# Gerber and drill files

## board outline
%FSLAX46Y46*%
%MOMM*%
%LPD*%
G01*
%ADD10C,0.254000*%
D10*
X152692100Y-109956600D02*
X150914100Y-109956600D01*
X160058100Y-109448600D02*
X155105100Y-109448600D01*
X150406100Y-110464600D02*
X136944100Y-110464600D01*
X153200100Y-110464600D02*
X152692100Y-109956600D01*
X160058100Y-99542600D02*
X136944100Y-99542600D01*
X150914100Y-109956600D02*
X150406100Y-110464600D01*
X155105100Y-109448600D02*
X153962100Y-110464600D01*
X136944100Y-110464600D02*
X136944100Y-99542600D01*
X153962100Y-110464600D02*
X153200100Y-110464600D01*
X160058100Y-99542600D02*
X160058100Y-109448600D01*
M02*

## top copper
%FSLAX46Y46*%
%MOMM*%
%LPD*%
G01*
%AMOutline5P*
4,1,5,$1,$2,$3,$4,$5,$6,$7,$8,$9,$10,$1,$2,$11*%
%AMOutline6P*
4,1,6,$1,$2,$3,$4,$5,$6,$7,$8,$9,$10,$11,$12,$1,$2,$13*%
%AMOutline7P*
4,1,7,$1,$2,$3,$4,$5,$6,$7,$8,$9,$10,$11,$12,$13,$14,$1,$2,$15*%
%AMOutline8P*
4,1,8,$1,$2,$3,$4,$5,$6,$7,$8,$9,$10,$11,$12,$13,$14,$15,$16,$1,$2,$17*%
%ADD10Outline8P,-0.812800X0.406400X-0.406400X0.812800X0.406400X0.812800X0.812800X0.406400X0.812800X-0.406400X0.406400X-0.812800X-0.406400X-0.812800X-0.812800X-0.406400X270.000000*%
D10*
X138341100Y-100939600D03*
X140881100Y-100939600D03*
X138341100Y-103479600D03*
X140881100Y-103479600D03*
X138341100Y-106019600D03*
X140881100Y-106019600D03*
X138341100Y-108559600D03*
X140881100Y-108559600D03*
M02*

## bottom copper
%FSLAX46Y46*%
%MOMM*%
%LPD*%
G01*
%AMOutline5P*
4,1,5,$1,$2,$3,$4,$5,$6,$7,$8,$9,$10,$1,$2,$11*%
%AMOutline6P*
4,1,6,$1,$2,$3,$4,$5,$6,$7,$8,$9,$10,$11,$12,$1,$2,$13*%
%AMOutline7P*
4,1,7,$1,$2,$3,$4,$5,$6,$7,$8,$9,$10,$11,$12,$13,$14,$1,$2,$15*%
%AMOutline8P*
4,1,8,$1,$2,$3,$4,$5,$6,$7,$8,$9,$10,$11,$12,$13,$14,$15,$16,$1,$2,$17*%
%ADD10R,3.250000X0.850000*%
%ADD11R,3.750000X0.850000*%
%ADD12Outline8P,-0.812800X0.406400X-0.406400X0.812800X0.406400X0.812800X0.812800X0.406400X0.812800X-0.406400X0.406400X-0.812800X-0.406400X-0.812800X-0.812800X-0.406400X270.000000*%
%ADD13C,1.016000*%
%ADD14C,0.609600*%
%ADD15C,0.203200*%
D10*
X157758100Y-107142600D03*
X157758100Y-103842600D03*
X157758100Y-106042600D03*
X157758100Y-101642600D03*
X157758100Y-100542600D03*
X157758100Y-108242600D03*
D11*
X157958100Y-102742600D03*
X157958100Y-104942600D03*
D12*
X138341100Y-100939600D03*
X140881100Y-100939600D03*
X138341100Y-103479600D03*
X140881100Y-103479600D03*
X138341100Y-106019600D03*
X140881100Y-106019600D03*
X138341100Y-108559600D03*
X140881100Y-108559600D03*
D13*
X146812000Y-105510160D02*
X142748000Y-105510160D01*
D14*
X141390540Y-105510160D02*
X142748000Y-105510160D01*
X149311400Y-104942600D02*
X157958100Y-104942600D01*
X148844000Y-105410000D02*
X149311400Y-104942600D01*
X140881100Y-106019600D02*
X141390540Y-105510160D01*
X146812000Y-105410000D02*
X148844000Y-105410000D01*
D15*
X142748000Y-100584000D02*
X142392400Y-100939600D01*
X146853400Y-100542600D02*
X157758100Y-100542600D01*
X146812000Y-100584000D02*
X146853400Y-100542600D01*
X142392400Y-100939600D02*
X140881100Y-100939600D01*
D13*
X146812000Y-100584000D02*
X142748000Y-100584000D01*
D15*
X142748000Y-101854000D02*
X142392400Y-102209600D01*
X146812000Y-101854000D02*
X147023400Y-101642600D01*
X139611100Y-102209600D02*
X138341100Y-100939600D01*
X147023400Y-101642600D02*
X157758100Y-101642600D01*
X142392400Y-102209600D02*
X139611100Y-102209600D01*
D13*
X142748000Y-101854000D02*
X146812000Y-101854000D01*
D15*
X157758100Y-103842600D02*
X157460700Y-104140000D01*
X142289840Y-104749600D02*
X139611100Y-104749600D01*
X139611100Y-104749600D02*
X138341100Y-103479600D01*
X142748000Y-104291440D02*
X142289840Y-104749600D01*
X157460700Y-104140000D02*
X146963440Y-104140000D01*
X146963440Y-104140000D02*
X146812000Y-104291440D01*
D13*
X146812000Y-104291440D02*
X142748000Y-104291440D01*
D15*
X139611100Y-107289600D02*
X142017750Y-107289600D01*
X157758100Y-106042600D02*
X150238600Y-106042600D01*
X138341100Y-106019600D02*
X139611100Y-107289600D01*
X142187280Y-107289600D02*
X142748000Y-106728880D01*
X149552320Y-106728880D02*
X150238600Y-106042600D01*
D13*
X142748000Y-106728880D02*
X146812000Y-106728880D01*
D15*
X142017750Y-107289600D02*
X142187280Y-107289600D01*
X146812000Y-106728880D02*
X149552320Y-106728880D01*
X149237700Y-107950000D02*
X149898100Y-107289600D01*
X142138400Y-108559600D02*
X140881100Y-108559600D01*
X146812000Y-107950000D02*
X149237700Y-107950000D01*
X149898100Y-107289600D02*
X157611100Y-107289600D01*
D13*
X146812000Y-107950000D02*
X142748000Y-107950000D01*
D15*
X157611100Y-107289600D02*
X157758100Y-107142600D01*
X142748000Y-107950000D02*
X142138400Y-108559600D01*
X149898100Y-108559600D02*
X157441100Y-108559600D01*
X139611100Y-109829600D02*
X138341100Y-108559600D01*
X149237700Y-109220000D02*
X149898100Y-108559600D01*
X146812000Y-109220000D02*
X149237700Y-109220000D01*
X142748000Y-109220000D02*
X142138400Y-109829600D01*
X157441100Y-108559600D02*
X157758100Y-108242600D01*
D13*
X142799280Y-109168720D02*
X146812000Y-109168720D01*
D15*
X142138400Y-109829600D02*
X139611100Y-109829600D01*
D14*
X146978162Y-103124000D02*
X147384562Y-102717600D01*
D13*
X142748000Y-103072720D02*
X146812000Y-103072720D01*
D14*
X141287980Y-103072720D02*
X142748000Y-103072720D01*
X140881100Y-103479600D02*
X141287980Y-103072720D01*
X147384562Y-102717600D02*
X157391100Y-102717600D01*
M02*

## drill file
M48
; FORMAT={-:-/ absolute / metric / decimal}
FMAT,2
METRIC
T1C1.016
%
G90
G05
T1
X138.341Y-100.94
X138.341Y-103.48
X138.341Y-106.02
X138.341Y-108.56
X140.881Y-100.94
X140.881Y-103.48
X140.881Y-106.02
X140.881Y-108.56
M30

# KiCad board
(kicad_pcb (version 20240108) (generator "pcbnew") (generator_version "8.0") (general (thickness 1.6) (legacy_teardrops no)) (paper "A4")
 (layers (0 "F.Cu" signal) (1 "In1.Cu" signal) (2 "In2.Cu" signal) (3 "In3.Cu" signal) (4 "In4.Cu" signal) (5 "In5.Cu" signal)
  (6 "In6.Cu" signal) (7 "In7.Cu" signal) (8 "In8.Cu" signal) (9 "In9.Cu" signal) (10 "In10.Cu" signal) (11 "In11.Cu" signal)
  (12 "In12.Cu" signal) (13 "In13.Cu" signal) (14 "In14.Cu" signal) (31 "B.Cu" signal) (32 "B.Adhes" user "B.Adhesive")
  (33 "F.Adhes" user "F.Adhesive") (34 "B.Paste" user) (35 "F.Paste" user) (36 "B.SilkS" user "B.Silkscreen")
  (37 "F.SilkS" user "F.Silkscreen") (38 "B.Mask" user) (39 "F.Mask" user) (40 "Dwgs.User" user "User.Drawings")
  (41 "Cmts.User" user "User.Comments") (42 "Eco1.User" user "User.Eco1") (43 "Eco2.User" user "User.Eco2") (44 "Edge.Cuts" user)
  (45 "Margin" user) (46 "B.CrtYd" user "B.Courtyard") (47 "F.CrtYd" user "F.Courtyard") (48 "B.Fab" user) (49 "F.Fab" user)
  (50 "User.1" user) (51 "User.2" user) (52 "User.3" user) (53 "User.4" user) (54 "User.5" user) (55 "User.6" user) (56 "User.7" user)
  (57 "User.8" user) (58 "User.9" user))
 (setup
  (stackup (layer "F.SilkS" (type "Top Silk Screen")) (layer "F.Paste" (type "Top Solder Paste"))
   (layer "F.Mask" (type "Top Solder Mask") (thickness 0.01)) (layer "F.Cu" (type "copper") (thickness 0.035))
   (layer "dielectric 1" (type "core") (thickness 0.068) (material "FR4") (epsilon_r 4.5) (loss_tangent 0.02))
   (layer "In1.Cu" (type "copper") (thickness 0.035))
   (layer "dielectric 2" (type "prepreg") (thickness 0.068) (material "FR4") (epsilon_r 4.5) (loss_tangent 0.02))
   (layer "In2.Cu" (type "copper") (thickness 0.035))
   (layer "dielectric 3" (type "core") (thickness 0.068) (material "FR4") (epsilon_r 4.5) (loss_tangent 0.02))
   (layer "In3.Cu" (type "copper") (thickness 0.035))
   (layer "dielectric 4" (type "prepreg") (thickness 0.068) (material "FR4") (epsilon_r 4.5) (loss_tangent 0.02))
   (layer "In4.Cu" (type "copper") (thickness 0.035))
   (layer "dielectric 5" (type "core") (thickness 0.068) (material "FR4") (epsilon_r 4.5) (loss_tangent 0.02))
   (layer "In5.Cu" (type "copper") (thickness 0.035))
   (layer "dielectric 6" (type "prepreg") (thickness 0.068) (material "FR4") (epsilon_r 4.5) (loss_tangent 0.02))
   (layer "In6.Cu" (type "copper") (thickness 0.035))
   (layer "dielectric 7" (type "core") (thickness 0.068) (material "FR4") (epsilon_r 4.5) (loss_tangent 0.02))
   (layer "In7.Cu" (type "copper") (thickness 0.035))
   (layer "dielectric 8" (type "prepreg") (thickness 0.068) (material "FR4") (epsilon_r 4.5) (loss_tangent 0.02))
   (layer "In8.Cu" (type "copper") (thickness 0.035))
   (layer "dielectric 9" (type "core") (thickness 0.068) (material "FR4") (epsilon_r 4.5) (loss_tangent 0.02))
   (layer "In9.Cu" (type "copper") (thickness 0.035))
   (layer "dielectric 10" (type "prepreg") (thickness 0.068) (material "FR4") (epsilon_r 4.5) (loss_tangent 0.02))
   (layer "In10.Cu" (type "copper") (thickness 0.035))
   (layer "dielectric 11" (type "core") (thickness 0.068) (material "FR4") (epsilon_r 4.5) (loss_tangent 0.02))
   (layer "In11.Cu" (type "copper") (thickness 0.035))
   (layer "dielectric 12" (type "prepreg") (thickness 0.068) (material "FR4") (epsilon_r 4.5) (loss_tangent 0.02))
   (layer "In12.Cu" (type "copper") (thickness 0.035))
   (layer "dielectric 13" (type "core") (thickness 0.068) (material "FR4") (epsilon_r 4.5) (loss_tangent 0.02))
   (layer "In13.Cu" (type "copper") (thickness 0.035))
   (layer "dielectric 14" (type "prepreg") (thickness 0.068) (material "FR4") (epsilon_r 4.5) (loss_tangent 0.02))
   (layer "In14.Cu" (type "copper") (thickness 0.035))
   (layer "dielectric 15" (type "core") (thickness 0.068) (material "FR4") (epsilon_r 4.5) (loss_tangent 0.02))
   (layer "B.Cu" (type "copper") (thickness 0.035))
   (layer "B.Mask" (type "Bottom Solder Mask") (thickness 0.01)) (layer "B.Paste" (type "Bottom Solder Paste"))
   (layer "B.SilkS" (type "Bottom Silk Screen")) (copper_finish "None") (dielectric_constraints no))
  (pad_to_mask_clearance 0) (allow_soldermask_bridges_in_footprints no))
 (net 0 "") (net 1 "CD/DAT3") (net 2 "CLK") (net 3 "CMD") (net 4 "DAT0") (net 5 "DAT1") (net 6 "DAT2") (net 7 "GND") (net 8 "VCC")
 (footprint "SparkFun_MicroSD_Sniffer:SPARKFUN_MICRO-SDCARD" (layer "F.Cu") (at 160.0581 109.7026 90)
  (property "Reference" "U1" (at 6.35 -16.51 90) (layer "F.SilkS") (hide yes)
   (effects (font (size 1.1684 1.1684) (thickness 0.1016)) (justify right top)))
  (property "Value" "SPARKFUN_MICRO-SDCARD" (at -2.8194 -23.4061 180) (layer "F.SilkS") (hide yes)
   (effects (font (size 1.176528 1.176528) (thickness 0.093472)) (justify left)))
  (pad "CD/DAT3" smd rect (at 2.56 -2.3 90) (size 0.85 3.25) (layers "B.Cu" "B.Paste" "B.Mask") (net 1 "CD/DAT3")
   (solder_mask_margin 0.1016))
  (pad "CLK" smd rect (at 5.86 -2.3 90) (size 0.85 3.25) (layers "B.Cu" "B.Paste" "B.Mask") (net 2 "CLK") (solder_mask_margin 0.1016))
  (pad "CMD" smd rect (at 3.66 -2.3 90) (size 0.85 3.25) (layers "B.Cu" "B.Paste" "B.Mask") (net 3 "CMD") (solder_mask_margin 0.1016))
  (pad "DAT0" smd rect (at 8.06 -2.3 90) (size 0.85 3.25) (layers "B.Cu" "B.Paste" "B.Mask") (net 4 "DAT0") (solder_mask_margin 0.1016))
  (pad "DAT1" smd rect (at 9.16 -2.3 90) (size 0.85 3.25) (layers "B.Cu" "B.Paste" "B.Mask") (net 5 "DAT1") (solder_mask_margin 0.1016))
  (pad "DAT2" smd rect (at 1.46 -2.3 90) (size 0.85 3.25) (layers "B.Cu" "B.Paste" "B.Mask") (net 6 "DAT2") (solder_mask_margin 0.1016))
  (pad "GND" smd rect (at 6.96 -2.1 270) (size 0.85 3.75) (layers "B.Cu" "B.Paste" "B.Mask") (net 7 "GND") (solder_mask_margin 0.1016))
  (pad "VCC" smd rect (at 4.76 -2.1 90) (size 0.85 3.75) (layers "B.Cu" "B.Paste" "B.Mask") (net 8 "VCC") (solder_mask_margin 0.1016)))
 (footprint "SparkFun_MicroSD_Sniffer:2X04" (layer "F.Cu") (at 139.6111 104.7496 -90)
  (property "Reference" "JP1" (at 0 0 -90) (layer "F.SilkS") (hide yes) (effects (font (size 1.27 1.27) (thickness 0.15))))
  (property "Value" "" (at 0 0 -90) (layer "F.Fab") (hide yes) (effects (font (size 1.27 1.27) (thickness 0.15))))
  (pad "1" thru_hole roundrect (at -3.81 1.27 270) (size 1.6256 1.6256) (drill 1.016) (layers "*.Cu" "*.Mask") (remove_unused_layers no)
   (roundrect_rratio 0.25) (chamfer_ratio 0.25) (chamfer top_left top_right bottom_left bottom_right) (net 4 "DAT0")
   (solder_mask_margin 0.1016))
  (pad "2" thru_hole roundrect (at -3.81 -1.27 270) (size 1.6256 1.6256) (drill 1.016) (layers "*.Cu" "*.Mask") (remove_unused_layers no)
   (roundrect_rratio 0.25) (chamfer_ratio 0.25) (chamfer top_left top_right bottom_left bottom_right) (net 5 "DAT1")
   (solder_mask_margin 0.1016))
  (pad "3" thru_hole roundrect (at -1.27 1.27 270) (size 1.6256 1.6256) (drill 1.016) (layers "*.Cu" "*.Mask") (remove_unused_layers no)
   (roundrect_rratio 0.25) (chamfer_ratio 0.25) (chamfer top_left top_right bottom_left bottom_right) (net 2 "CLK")
   (solder_mask_margin 0.1016))
  (pad "4" thru_hole roundrect (at -1.27 -1.27 270) (size 1.6256 1.6256) (drill 1.016) (layers "*.Cu" "*.Mask") (remove_unused_layers no)
   (roundrect_rratio 0.25) (chamfer_ratio 0.25) (chamfer top_left top_right bottom_left bottom_right) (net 7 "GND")
   (solder_mask_margin 0.1016))
  (pad "5" thru_hole roundrect (at 1.27 1.27 270) (size 1.6256 1.6256) (drill 1.016) (layers "*.Cu" "*.Mask") (remove_unused_layers no)
   (roundrect_rratio 0.25) (chamfer_ratio 0.25) (chamfer top_left top_right bottom_left bottom_right) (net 3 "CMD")
   (solder_mask_margin 0.1016))
  (pad "6" thru_hole roundrect (at 1.27 -1.27 270) (size 1.6256 1.6256) (drill 1.016) (layers "*.Cu" "*.Mask") (remove_unused_layers no)
   (roundrect_rratio 0.25) (chamfer_ratio 0.25) (chamfer top_left top_right bottom_left bottom_right) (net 8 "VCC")
   (solder_mask_margin 0.1016))
  (pad "7" thru_hole roundrect (at 3.81 1.27 270) (size 1.6256 1.6256) (drill 1.016) (layers "*.Cu" "*.Mask") (remove_unused_layers no)
   (roundrect_rratio 0.25) (chamfer_ratio 0.25) (chamfer top_left top_right bottom_left bottom_right) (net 6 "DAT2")
   (solder_mask_margin 0.1016))
  (pad "8" thru_hole roundrect (at 3.81 -1.27 270) (size 1.6256 1.6256) (drill 1.016) (layers "*.Cu" "*.Mask") (remove_unused_layers no)
   (roundrect_rratio 0.25) (chamfer_ratio 0.25) (chamfer top_left top_right bottom_left bottom_right) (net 1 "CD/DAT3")
   (solder_mask_margin 0.1016)))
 (gr_line (start 152.6921 109.9566) (end 150.9141 109.9566) (stroke (width 0.254) (type solid)) (layer "Edge.Cuts"))
 (gr_line (start 160.0581 109.4486) (end 155.1051 109.4486) (stroke (width 0.254) (type solid)) (layer "Edge.Cuts"))
 (gr_line (start 150.4061 110.4646) (end 136.9441 110.4646) (stroke (width 0.254) (type solid)) (layer "Edge.Cuts"))
 (gr_line (start 153.2001 110.4646) (end 152.6921 109.9566) (stroke (width 0.254) (type solid)) (layer "Edge.Cuts"))
 (gr_line (start 160.0581 99.5426) (end 136.9441 99.5426) (stroke (width 0.254) (type solid)) (layer "Edge.Cuts"))
 (gr_line (start 150.9141 109.9566) (end 150.4061 110.4646) (stroke (width 0.254) (type solid)) (layer "Edge.Cuts"))
 (gr_line (start 155.1051 109.4486) (end 153.9621 110.4646) (stroke (width 0.254) (type solid)) (layer "Edge.Cuts"))
 (gr_line (start 136.9441 110.4646) (end 136.9441 99.5426) (stroke (width 0.254) (type solid)) (layer "Edge.Cuts"))
 (gr_line (start 153.9621 110.4646) (end 153.2001 110.4646) (stroke (width 0.254) (type solid)) (layer "Edge.Cuts"))
 (gr_line (start 160.0581 99.5426) (end 160.0581 109.4486) (stroke (width 0.254) (type solid)) (layer "Edge.Cuts"))
 (segment (start 146.812 105.51016) (end 142.748 105.51016) (width 1.016) (layer "B.Cu") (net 8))
 (segment (start 141.39054 105.51016) (end 142.748 105.51016) (width 0.6096) (layer "B.Cu") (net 8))
 (segment (start 149.3114 104.9426) (end 157.9581 104.9426) (width 0.6096) (layer "B.Cu") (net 8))
 (segment (start 148.844 105.41) (end 149.3114 104.9426) (width 0.6096) (layer "B.Cu") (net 8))
 (segment (start 140.8811 106.0196) (end 141.39054 105.51016) (width 0.6096) (layer "B.Cu") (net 8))
 (segment (start 146.812 105.41) (end 148.844 105.41) (width 0.6096) (layer "B.Cu") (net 8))
 (segment (start 142.748 100.584) (end 142.3924 100.9396) (width 0.2032) (layer "B.Cu") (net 5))
 (segment (start 146.8534 100.5426) (end 157.7581 100.5426) (width 0.2032) (layer "B.Cu") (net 5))
 (segment (start 146.812 100.584) (end 146.8534 100.5426) (width 0.2032) (layer "B.Cu") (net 5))
 (segment (start 142.3924 100.9396) (end 140.8811 100.9396) (width 0.2032) (layer "B.Cu") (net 5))
 (segment (start 146.812 100.584) (end 142.748 100.584) (width 1.016) (layer "B.Cu") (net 5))
 (segment (start 142.748 101.854) (end 142.3924 102.2096) (width 0.2032) (layer "B.Cu") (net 4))
 (segment (start 146.812 101.854) (end 147.0234 101.6426) (width 0.2032) (layer "B.Cu") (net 4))
 (segment (start 139.6111 102.2096) (end 138.3411 100.9396) (width 0.2032) (layer "B.Cu") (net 4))
 (segment (start 147.0234 101.6426) (end 157.7581 101.6426) (width 0.2032) (layer "B.Cu") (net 4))
 (segment (start 142.3924 102.2096) (end 139.6111 102.2096) (width 0.2032) (layer "B.Cu") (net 4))
 (segment (start 142.748 101.854) (end 146.812 101.854) (width 1.016) (layer "B.Cu") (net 4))
 (segment (start 157.7581 103.8426) (end 157.4607 104.14) (width 0.2032) (layer "B.Cu") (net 2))
 (segment (start 142.28984 104.7496) (end 139.6111 104.7496) (width 0.2032) (layer "B.Cu") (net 2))
 (segment (start 139.6111 104.7496) (end 138.3411 103.4796) (width 0.2032) (layer "B.Cu") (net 2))
 (segment (start 142.748 104.29144) (end 142.28984 104.7496) (width 0.2032) (layer "B.Cu") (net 2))
 (segment (start 157.4607 104.14) (end 146.96344 104.14) (width 0.2032) (layer "B.Cu") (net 2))
 (segment (start 146.96344 104.14) (end 146.812 104.29144) (width 0.2032) (layer "B.Cu") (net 2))
 (segment (start 146.812 104.29144) (end 142.748 104.29144) (width 1.016) (layer "B.Cu") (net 2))
 (segment (start 139.6111 107.2896) (end 142.01775 107.2896) (width 0.2032) (layer "B.Cu") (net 3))
 (segment (start 157.7581 106.0426) (end 150.2386 106.0426) (width 0.2032) (layer "B.Cu") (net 3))
 (segment (start 138.3411 106.0196) (end 139.6111 107.2896) (width 0.2032) (layer "B.Cu") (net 3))
 (segment (start 142.18728 107.2896) (end 142.748 106.72888) (width 0.2032) (layer "B.Cu") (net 3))
 (segment (start 149.55232 106.72888) (end 150.2386 106.0426) (width 0.2032) (layer "B.Cu") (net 3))
 (segment (start 142.748 106.72888) (end 146.812 106.72888) (width 1.016) (layer "B.Cu") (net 3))
 (segment (start 142.01775 107.2896) (end 142.18728 107.2896) (width 0.2032) (layer "B.Cu") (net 3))
 (segment (start 146.812 106.72888) (end 149.55232 106.72888) (width 0.2032) (layer "B.Cu") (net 3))
 (segment (start 149.2377 107.95) (end 149.8981 107.2896) (width 0.2032) (layer "B.Cu") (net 1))
 (segment (start 142.1384 108.5596) (end 140.8811 108.5596) (width 0.2032) (layer "B.Cu") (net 1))
 (segment (start 146.812 107.95) (end 149.2377 107.95) (width 0.2032) (layer "B.Cu") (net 1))
 (segment (start 149.8981 107.2896) (end 157.6111 107.2896) (width 0.2032) (layer "B.Cu") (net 1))
 (segment (start 146.812 107.95) (end 142.748 107.95) (width 1.016) (layer "B.Cu") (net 1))
 (segment (start 157.6111 107.2896) (end 157.7581 107.1426) (width 0.2032) (layer "B.Cu") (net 1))
 (segment (start 142.748 107.95) (end 142.1384 108.5596) (width 0.2032) (layer "B.Cu") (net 1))
 (segment (start 149.8981 108.5596) (end 157.4411 108.5596) (width 0.2032) (layer "B.Cu") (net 6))
 (segment (start 139.6111 109.8296) (end 138.3411 108.5596) (width 0.2032) (layer "B.Cu") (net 6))
 (segment (start 149.2377 109.22) (end 149.8981 108.5596) (width 0.2032) (layer "B.Cu") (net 6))
 (segment (start 146.812 109.22) (end 149.2377 109.22) (width 0.2032) (layer "B.Cu") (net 6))
 (segment (start 142.748 109.22) (end 142.1384 109.8296) (width 0.2032) (layer "B.Cu") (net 6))
 (segment (start 157.4411 108.5596) (end 157.7581 108.2426) (width 0.2032) (layer "B.Cu") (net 6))
 (segment (start 142.79928 109.16872) (end 146.812 109.16872) (width 1.016) (layer "B.Cu") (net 6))
 (segment (start 142.1384 109.8296) (end 139.6111 109.8296) (width 0.2032) (layer "B.Cu") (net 6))
 (segment (start 146.978162 103.124) (end 147.384562 102.7176) (width 0.6096) (layer "B.Cu") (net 7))
 (segment (start 142.748 103.07272) (end 146.812 103.07272) (width 1.016) (layer "B.Cu") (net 7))
 (segment (start 141.28798 103.07272) (end 142.748 103.07272) (width 0.6096) (layer "B.Cu") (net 7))
 (segment (start 140.8811 103.4796) (end 141.28798 103.07272) (width 0.6096) (layer "B.Cu") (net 7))
 (segment (start 147.384562 102.7176) (end 157.3911 102.7176) (width 0.6096) (layer "B.Cu") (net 7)))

